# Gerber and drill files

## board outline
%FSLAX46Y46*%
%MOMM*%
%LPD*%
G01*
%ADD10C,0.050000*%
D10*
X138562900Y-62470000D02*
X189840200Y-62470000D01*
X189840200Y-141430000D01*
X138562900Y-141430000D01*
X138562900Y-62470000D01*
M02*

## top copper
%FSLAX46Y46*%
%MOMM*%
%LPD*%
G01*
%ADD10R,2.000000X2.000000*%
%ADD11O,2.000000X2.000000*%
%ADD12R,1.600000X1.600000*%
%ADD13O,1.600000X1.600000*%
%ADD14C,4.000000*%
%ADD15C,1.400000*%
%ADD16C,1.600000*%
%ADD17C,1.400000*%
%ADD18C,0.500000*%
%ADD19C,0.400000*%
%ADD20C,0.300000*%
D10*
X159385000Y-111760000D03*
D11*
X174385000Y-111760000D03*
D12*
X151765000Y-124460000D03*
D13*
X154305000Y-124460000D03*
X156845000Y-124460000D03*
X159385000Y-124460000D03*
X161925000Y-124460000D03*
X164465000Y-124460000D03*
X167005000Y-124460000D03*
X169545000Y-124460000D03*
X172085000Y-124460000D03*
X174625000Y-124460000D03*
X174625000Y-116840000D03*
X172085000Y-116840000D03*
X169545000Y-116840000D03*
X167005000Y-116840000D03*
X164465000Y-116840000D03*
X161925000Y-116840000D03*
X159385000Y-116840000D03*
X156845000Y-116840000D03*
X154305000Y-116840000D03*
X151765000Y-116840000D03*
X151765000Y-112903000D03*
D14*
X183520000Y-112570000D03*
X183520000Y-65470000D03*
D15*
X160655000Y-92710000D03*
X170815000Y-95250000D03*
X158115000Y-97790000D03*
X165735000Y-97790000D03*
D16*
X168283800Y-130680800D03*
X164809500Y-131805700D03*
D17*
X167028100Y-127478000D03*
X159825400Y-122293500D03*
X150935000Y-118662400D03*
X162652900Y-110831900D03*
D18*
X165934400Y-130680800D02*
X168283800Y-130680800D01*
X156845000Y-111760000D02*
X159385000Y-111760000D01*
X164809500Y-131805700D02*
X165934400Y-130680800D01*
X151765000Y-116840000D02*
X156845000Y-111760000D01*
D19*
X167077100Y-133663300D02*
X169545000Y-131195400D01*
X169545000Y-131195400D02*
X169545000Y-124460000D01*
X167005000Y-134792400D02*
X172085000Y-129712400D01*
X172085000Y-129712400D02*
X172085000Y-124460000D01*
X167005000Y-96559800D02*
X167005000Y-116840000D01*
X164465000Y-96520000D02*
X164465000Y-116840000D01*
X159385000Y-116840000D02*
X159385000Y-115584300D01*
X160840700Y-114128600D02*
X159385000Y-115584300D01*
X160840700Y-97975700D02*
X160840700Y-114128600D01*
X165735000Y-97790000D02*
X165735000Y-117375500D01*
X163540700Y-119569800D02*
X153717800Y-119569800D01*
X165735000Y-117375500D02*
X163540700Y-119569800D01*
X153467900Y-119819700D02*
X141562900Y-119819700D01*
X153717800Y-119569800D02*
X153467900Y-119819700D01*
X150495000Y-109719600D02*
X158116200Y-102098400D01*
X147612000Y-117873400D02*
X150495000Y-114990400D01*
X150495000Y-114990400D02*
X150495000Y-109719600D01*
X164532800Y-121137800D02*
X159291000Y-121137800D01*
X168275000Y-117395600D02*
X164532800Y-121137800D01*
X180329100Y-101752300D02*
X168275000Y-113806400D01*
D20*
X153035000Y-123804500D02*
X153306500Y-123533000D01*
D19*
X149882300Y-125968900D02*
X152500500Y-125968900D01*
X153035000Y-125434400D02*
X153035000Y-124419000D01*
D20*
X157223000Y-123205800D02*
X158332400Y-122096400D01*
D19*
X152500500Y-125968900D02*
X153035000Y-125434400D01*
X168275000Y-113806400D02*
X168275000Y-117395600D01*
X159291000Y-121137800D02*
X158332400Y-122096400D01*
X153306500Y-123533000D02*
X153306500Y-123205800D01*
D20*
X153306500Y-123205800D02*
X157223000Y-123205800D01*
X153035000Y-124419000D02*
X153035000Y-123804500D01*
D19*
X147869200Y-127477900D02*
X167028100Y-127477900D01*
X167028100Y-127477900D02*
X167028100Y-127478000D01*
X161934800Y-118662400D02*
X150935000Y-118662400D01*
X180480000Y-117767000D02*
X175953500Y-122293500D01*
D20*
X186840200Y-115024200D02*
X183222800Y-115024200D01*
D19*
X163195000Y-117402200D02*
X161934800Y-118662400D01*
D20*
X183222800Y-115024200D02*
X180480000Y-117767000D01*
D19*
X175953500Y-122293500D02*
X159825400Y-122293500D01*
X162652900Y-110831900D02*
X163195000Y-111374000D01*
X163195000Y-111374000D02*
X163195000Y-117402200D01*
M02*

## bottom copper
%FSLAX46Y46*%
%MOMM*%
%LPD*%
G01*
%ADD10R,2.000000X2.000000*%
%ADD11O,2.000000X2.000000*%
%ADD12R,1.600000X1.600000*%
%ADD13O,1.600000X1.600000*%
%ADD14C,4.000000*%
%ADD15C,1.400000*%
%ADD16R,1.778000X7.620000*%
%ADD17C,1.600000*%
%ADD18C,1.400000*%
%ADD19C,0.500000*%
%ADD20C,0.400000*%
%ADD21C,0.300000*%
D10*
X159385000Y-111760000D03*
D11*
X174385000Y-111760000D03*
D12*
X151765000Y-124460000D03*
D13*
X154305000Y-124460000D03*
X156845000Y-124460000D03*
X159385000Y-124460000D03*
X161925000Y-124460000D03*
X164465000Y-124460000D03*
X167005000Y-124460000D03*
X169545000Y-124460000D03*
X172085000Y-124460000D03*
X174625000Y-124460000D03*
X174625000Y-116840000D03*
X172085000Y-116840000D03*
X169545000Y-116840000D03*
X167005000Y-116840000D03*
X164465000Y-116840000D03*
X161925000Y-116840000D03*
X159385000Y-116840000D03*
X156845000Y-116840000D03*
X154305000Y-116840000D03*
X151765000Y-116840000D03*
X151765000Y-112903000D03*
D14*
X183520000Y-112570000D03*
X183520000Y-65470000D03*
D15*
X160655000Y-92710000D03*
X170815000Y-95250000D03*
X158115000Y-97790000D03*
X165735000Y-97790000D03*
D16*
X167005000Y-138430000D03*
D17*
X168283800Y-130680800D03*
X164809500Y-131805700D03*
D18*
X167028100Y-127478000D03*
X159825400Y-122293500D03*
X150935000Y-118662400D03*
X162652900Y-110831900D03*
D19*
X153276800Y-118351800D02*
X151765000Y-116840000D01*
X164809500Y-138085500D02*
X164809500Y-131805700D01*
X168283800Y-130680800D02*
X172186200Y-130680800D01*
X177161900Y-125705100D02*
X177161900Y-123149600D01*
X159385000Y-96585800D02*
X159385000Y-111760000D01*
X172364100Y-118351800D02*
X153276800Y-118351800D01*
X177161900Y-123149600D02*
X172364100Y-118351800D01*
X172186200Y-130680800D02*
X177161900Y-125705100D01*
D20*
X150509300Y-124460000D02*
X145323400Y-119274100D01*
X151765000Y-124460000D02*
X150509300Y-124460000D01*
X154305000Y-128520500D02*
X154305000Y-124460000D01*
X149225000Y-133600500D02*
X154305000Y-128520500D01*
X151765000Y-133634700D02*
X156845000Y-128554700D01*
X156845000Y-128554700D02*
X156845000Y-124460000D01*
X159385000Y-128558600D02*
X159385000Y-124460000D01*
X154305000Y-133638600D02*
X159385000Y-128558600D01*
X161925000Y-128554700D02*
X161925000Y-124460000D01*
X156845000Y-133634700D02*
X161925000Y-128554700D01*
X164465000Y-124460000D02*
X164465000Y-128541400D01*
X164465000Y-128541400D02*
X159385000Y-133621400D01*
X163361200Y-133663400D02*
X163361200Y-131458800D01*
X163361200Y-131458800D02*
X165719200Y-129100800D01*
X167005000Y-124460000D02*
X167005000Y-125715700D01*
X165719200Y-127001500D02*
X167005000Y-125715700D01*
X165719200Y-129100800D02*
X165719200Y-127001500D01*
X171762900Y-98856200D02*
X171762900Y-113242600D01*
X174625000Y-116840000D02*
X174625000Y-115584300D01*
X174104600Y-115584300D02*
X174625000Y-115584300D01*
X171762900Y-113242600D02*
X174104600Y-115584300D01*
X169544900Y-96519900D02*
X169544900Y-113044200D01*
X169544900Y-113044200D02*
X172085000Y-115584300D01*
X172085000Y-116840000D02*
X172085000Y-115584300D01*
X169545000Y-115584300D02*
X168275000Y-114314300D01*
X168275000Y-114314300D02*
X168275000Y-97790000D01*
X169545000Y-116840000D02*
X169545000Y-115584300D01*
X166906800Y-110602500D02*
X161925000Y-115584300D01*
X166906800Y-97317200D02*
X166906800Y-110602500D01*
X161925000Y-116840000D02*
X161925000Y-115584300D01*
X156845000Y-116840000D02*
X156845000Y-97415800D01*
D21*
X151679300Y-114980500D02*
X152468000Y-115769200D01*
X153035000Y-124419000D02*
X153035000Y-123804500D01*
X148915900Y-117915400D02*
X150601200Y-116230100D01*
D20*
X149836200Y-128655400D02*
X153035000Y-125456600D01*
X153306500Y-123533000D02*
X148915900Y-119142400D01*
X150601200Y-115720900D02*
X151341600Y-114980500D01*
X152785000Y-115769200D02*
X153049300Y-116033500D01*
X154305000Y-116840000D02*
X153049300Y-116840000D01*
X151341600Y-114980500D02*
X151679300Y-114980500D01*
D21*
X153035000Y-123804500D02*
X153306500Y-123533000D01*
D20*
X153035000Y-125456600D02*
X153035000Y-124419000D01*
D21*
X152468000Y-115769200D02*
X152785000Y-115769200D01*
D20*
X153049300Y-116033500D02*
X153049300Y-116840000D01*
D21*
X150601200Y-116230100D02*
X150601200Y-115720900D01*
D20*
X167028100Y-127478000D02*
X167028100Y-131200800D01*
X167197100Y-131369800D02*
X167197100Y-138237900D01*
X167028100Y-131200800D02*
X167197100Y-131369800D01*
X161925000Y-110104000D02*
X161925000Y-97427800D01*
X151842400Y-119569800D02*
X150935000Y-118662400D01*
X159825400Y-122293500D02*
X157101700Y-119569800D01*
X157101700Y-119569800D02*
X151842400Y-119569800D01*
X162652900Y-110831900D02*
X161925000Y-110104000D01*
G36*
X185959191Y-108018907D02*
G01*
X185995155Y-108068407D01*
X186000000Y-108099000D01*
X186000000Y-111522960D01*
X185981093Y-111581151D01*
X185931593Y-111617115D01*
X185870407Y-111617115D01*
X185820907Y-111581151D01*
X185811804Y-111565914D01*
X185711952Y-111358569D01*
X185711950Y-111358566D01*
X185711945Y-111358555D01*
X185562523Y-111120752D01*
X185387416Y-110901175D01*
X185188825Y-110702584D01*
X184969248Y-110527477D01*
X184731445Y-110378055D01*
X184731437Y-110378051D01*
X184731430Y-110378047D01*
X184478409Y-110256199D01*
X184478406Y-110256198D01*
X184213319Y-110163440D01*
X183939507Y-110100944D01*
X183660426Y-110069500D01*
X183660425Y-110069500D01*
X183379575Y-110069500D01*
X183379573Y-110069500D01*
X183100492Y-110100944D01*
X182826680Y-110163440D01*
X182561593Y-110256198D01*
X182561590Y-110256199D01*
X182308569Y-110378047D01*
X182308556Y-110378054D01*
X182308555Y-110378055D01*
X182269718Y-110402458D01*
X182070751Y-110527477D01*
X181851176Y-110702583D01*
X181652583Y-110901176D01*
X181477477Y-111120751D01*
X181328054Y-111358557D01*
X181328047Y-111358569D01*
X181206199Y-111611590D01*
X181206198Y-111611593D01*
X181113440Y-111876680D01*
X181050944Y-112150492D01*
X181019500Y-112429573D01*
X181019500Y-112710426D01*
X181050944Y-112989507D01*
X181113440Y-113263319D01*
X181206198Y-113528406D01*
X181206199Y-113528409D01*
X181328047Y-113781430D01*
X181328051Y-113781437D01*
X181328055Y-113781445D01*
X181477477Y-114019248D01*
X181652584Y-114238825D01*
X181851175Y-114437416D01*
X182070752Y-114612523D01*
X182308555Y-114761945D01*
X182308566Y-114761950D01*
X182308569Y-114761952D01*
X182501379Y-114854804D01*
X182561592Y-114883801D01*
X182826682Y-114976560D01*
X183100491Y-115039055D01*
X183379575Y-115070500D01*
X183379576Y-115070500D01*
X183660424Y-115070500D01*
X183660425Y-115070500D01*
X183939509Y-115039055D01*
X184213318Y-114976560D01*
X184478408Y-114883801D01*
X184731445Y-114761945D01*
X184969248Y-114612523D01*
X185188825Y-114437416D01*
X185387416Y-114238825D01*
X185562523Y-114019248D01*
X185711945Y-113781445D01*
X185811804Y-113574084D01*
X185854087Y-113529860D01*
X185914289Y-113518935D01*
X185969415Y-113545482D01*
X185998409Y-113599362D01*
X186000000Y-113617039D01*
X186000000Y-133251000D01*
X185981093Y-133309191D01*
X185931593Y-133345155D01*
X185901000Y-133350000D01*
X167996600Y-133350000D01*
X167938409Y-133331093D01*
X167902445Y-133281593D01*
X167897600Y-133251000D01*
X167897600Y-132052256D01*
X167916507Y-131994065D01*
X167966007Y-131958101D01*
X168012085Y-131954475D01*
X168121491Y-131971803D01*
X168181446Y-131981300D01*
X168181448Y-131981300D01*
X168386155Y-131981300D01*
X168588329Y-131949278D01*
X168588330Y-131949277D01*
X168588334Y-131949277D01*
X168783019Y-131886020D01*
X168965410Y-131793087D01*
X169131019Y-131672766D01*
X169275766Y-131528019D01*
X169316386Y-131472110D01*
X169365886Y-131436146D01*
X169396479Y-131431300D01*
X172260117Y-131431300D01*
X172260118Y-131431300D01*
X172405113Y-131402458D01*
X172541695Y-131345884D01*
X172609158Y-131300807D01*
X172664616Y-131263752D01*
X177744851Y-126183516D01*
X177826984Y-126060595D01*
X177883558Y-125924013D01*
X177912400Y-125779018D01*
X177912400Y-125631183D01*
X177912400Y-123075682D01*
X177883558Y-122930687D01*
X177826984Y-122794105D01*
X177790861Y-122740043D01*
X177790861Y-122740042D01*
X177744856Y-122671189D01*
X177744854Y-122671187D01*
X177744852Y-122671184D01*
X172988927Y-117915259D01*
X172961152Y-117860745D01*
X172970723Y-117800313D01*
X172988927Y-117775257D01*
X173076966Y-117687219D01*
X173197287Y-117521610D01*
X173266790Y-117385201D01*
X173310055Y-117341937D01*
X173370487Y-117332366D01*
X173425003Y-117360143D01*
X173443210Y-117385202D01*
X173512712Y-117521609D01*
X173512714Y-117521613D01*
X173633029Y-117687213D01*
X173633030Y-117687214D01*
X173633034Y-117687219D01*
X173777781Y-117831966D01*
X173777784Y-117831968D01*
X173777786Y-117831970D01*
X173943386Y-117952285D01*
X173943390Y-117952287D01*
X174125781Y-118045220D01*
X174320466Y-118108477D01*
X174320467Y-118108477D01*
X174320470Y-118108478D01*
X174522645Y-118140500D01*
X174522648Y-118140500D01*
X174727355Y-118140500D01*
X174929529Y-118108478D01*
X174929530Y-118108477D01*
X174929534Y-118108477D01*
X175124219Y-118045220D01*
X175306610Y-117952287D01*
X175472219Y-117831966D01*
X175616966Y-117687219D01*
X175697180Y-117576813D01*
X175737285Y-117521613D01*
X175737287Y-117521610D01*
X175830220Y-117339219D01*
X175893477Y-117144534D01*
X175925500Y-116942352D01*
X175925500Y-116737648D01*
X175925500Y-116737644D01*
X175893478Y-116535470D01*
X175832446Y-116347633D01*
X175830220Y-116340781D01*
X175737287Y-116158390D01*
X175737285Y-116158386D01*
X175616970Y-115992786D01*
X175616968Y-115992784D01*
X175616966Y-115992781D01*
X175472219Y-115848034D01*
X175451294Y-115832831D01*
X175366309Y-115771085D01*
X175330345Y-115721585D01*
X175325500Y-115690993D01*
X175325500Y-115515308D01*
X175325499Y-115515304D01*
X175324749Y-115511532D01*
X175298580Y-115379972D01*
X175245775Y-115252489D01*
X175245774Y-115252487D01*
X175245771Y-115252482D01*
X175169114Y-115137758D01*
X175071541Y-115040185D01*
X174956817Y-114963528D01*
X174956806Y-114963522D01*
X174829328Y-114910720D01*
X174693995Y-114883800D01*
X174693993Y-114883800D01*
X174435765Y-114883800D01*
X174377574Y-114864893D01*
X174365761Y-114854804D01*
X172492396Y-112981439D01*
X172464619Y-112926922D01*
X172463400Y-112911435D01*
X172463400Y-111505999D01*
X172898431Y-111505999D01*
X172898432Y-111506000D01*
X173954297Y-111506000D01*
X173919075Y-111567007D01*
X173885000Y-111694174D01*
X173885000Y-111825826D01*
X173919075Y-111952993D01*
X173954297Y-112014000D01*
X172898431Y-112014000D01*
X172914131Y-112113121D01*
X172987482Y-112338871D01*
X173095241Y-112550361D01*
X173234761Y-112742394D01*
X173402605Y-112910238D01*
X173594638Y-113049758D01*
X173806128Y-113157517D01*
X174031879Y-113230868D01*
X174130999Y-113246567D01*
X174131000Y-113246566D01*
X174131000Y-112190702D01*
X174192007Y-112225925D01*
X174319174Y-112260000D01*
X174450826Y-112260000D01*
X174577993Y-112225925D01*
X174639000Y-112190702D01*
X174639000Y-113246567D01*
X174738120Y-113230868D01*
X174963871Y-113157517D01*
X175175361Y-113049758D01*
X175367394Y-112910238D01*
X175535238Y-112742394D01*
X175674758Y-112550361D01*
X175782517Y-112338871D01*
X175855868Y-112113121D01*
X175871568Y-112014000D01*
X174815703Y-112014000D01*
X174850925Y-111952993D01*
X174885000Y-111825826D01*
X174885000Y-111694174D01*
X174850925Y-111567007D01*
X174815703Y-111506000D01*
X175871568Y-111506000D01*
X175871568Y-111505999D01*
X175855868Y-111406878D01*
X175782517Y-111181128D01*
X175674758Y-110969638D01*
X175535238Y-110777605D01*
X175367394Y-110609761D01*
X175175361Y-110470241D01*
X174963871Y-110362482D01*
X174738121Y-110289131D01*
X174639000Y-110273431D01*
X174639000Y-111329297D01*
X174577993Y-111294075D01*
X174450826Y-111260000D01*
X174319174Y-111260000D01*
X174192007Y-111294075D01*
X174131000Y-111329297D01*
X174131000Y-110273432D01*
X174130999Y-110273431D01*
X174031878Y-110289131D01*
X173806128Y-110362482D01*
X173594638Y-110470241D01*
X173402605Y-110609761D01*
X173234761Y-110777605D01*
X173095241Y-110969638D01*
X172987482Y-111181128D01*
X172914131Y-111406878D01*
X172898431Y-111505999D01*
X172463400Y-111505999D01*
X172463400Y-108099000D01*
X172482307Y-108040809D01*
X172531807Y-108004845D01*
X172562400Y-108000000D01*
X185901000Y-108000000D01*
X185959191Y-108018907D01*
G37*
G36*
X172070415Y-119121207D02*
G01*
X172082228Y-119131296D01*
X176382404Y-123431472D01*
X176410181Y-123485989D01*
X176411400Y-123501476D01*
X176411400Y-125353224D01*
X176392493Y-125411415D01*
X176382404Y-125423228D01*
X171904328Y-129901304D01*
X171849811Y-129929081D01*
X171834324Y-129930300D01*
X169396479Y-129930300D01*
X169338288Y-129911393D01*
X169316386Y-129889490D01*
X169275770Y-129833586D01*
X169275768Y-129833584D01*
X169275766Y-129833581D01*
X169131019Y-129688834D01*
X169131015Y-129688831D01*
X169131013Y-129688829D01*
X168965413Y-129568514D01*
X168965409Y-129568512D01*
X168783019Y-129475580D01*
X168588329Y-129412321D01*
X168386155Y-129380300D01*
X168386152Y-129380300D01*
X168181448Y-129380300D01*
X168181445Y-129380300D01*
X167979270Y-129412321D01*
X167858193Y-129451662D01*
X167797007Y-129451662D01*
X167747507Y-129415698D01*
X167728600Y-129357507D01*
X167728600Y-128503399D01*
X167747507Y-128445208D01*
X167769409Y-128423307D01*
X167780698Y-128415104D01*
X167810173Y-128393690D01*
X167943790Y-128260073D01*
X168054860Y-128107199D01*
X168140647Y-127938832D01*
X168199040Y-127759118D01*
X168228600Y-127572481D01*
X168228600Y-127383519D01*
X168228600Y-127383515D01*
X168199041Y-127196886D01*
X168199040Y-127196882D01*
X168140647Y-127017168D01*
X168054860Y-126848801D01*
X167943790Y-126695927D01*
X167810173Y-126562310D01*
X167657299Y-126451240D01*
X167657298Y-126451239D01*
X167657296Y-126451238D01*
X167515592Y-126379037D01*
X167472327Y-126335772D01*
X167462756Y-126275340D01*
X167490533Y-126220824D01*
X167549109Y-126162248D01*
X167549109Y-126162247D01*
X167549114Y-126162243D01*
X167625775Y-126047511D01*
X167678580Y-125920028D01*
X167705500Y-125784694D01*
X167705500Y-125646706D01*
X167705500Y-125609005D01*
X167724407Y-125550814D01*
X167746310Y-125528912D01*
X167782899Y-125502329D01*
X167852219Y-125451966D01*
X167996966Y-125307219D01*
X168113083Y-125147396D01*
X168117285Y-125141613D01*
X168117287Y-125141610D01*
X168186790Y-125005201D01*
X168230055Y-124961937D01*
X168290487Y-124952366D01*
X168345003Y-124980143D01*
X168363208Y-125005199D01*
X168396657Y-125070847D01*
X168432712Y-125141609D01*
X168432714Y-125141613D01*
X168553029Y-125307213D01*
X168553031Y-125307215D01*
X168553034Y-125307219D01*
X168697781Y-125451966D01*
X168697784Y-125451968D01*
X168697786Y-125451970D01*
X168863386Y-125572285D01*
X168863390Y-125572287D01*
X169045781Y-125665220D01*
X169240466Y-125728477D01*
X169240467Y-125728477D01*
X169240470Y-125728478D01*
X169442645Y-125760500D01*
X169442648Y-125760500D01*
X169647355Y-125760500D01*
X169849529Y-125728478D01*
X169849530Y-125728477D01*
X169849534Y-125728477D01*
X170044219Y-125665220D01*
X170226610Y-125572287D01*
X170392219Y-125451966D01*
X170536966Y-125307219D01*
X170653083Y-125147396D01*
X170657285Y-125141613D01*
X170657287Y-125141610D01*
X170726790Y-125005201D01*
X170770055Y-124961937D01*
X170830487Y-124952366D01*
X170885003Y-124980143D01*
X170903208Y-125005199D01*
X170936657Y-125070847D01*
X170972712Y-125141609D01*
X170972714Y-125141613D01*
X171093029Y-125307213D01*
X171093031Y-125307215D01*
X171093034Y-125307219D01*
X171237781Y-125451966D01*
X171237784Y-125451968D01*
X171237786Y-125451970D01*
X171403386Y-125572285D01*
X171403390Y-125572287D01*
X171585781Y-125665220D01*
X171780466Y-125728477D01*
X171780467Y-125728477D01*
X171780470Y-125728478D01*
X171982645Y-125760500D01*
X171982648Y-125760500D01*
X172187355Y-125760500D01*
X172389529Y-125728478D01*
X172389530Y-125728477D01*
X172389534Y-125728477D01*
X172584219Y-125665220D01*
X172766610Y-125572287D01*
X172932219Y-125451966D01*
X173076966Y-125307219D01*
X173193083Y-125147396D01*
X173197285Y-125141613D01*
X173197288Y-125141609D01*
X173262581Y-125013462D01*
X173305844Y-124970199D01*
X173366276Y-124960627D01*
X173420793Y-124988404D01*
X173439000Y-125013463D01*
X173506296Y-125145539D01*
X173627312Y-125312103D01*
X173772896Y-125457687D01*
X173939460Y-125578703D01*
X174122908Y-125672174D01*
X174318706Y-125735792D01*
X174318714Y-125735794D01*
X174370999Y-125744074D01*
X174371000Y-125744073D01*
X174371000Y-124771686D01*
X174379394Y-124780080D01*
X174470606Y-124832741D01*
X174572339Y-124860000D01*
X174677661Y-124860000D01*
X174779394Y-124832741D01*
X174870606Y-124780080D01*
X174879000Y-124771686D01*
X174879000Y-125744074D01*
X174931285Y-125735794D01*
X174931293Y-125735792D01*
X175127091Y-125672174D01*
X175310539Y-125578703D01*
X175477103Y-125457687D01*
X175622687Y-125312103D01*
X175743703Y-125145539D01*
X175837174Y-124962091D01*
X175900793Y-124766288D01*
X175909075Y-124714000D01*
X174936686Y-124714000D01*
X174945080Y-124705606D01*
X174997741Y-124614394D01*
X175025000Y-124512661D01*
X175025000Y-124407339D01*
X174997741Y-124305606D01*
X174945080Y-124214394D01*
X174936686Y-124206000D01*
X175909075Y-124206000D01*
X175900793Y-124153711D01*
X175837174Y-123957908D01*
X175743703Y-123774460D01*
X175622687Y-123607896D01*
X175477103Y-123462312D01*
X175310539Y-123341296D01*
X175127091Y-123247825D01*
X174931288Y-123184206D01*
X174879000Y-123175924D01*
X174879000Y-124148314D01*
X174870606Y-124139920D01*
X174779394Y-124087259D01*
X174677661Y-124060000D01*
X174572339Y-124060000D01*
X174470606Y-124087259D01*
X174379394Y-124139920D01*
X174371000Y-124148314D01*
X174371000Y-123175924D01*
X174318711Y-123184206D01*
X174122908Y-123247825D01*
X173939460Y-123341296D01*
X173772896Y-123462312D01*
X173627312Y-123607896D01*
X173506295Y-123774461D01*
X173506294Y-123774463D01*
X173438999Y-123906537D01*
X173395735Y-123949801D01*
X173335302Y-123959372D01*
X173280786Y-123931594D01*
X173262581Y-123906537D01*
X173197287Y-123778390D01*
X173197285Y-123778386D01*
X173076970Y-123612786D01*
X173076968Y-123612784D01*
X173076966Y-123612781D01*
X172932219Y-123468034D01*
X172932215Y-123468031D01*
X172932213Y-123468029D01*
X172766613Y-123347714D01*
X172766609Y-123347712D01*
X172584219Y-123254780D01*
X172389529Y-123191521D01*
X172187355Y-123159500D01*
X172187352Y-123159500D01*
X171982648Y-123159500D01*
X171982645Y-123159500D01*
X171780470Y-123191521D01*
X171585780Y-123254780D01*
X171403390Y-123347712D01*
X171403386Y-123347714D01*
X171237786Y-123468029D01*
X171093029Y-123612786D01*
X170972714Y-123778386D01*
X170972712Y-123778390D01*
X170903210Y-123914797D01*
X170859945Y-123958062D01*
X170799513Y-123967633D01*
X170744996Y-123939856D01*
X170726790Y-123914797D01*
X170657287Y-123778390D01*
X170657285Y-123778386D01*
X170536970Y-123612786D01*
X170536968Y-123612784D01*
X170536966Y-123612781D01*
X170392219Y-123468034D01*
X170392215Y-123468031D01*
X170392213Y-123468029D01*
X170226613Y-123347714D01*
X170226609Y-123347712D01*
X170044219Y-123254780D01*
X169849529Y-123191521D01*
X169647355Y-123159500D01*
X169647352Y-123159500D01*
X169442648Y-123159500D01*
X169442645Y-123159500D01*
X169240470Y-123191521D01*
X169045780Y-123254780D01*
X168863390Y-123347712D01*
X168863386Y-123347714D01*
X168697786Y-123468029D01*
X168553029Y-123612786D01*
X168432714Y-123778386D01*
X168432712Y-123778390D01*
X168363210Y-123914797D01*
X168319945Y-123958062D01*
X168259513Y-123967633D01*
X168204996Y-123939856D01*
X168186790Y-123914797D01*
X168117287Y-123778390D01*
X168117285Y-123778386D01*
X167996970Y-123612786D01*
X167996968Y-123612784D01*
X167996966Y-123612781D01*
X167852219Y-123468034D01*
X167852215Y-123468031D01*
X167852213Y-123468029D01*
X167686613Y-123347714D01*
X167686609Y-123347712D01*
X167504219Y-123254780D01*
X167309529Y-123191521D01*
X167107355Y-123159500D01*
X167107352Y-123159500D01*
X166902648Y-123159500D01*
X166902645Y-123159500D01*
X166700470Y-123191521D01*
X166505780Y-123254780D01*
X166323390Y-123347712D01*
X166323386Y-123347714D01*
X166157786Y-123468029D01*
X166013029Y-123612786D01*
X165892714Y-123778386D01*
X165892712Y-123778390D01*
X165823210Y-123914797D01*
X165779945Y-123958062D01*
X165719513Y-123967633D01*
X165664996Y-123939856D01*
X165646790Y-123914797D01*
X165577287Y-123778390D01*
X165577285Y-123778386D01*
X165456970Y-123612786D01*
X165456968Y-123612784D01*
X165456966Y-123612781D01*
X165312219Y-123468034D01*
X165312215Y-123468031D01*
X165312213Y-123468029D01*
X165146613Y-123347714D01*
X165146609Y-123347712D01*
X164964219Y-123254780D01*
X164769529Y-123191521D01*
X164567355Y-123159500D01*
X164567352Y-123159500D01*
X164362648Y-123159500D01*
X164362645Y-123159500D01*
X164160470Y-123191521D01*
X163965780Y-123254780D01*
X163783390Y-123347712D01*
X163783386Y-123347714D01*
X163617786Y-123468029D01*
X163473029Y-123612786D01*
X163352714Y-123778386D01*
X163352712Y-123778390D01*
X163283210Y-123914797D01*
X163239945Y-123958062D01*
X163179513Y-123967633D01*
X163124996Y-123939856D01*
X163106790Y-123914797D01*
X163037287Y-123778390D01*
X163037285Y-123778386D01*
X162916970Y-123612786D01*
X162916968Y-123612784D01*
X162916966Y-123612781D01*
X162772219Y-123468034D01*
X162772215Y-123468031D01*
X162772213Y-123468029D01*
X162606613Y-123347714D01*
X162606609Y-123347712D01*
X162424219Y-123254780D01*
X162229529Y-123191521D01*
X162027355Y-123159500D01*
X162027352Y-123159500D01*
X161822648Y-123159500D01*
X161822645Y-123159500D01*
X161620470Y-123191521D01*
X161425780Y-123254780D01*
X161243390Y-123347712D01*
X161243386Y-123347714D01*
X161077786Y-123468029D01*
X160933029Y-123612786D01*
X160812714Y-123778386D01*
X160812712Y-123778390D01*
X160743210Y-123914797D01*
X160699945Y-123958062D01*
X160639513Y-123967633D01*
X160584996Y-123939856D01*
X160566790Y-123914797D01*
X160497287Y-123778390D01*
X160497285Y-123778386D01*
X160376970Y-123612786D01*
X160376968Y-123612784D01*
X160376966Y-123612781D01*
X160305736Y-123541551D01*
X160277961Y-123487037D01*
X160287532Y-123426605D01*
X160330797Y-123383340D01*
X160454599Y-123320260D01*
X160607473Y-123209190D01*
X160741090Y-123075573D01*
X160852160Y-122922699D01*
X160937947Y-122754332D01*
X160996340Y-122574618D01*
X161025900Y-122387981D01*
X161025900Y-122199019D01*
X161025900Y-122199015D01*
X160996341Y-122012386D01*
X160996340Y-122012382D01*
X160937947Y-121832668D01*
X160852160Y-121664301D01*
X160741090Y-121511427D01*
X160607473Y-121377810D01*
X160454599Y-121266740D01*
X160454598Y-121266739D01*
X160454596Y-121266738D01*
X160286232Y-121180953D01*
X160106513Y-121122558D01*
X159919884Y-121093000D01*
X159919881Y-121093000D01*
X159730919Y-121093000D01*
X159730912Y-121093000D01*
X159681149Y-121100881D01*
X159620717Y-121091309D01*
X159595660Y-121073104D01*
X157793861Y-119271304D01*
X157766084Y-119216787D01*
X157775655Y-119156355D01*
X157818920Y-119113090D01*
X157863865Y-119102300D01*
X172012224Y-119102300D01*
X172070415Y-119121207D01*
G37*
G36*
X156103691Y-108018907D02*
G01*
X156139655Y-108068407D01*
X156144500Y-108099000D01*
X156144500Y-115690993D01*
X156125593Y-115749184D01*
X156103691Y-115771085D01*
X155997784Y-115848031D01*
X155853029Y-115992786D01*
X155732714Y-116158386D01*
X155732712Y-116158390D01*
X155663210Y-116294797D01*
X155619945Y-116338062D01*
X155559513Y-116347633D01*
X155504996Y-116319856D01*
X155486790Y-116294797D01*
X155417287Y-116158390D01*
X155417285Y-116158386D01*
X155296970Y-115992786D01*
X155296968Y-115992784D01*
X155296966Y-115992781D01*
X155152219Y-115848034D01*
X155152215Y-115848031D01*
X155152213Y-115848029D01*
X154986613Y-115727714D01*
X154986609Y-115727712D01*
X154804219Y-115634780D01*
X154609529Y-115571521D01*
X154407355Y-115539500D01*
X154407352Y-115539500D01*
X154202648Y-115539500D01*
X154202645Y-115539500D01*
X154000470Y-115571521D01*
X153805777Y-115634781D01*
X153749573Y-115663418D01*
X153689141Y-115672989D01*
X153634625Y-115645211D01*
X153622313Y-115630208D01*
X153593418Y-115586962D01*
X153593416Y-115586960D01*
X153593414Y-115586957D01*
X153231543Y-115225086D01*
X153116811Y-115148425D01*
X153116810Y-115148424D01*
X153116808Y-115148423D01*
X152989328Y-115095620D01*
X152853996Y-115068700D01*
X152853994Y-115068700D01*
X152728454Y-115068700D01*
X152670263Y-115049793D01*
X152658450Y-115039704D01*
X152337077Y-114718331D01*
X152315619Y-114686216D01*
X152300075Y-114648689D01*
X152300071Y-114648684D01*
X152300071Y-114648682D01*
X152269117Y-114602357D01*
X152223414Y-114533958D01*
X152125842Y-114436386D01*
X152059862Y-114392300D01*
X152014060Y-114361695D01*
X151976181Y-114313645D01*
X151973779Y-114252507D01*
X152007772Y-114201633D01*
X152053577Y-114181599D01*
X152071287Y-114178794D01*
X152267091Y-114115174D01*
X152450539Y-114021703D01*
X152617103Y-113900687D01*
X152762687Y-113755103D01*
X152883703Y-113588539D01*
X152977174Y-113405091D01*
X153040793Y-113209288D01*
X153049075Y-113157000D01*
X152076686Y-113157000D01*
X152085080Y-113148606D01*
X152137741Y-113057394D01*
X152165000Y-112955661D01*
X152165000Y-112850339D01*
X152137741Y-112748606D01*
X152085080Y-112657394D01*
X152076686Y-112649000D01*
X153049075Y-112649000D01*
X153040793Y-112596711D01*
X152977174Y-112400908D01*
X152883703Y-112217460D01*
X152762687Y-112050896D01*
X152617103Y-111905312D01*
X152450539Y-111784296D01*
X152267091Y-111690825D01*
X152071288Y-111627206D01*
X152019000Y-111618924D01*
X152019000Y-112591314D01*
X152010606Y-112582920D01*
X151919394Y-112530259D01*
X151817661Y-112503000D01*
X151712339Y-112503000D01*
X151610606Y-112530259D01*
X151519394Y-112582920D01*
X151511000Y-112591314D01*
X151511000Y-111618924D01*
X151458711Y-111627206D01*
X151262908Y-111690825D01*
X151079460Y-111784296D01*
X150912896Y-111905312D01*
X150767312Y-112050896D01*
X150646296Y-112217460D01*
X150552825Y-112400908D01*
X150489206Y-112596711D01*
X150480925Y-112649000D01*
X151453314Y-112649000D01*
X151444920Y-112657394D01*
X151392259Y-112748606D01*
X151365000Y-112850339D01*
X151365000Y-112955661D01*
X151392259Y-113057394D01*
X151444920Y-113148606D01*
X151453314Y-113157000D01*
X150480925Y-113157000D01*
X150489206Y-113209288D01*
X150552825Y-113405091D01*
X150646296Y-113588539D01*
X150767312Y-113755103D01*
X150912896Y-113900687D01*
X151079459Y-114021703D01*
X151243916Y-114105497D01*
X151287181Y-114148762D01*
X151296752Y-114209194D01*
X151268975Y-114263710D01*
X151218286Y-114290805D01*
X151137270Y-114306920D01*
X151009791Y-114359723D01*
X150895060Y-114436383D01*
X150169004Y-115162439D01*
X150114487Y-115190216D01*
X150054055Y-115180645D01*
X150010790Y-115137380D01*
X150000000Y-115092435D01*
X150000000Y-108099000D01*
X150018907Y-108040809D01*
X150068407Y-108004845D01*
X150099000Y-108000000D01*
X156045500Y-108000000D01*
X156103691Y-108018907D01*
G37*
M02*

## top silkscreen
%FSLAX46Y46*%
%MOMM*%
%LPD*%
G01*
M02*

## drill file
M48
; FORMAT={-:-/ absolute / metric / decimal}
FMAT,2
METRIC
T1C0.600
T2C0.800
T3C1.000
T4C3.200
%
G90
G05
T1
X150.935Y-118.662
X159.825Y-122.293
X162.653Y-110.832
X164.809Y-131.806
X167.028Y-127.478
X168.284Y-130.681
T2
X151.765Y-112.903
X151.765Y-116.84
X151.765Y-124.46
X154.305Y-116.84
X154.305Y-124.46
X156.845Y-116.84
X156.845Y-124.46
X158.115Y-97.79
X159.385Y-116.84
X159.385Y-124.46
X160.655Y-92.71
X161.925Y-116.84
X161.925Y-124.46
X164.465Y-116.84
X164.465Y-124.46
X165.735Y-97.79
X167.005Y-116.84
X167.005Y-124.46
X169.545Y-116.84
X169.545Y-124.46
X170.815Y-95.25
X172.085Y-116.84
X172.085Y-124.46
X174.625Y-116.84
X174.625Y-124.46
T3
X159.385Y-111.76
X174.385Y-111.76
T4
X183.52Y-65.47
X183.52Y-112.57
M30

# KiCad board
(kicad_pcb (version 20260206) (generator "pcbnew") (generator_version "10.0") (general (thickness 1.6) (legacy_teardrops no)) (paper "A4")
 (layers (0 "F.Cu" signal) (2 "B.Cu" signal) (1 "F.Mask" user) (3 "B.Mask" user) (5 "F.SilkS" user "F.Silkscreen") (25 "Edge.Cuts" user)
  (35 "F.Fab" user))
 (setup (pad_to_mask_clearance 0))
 (gr_rect (start 138.5629 62.47) (end 189.8402 141.43) (stroke (width 0.05) (type default)) (fill no) (layer "Edge.Cuts"))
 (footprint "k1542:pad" (layer "F.Cu") (at 159.385 111.76 0.0)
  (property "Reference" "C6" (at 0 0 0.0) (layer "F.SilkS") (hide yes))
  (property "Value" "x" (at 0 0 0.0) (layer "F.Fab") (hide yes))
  (pad "1" thru_hole rect (at 0 0 0.0) (size 2.0 2.0) (drill 1.0) (layers "*.Cu" "*.Mask") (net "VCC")))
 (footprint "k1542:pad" (layer "F.Cu") (at 174.385 111.76 0.0)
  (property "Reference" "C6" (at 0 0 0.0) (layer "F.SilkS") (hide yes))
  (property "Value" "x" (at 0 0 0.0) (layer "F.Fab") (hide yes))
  (pad "2" thru_hole oval (at 0 0 0.0) (size 2.0 2.0) (drill 1.0) (layers "*.Cu" "*.Mask") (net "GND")))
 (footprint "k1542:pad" (layer "F.Cu") (at 151.765 124.46 90.0)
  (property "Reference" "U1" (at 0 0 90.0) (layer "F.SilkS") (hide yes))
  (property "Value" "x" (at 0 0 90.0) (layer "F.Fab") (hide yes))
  (pad "1" thru_hole rect (at 0 0 90.0) (size 1.6 1.6) (drill 0.8) (layers "*.Cu" "*.Mask") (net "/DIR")))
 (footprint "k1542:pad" (layer "F.Cu") (at 154.305 124.46 90.0)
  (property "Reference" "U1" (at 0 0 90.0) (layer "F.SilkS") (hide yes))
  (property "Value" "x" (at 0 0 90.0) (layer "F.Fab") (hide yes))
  (pad "2" thru_hole oval (at 0 0 90.0) (size 1.6 1.6) (drill 0.8) (layers "*.Cu" "*.Mask") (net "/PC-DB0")))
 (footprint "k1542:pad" (layer "F.Cu") (at 156.845 124.46 90.0)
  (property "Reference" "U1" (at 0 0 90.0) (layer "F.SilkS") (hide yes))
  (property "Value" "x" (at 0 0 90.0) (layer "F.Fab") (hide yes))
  (pad "3" thru_hole oval (at 0 0 90.0) (size 1.6 1.6) (drill 0.8) (layers "*.Cu" "*.Mask") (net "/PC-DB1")))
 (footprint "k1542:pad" (layer "F.Cu") (at 159.385 124.46 90.0)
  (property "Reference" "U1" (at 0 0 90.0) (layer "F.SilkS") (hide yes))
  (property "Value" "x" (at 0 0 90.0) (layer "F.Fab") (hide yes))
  (pad "4" thru_hole oval (at 0 0 90.0) (size 1.6 1.6) (drill 0.8) (layers "*.Cu" "*.Mask") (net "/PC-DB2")))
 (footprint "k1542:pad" (layer "F.Cu") (at 161.925 124.46 90.0)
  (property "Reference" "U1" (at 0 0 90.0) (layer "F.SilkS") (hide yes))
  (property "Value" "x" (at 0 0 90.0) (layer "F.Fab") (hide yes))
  (pad "5" thru_hole oval (at 0 0 90.0) (size 1.6 1.6) (drill 0.8) (layers "*.Cu" "*.Mask") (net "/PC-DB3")))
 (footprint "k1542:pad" (layer "F.Cu") (at 164.465 124.46 90.0)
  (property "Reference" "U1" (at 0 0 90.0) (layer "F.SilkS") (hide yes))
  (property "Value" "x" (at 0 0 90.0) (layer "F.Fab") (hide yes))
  (pad "6" thru_hole oval (at 0 0 90.0) (size 1.6 1.6) (drill 0.8) (layers "*.Cu" "*.Mask") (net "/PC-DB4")))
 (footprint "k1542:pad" (layer "F.Cu") (at 167.005 124.46 90.0)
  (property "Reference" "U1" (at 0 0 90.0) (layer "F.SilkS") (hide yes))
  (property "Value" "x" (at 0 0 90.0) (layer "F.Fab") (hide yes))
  (pad "7" thru_hole oval (at 0 0 90.0) (size 1.6 1.6) (drill 0.8) (layers "*.Cu" "*.Mask") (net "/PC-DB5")))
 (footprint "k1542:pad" (layer "F.Cu") (at 169.545 124.46 90.0)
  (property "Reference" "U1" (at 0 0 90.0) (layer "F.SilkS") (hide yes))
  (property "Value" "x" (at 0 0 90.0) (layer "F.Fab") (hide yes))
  (pad "8" thru_hole oval (at 0 0 90.0) (size 1.6 1.6) (drill 0.8) (layers "*.Cu" "*.Mask") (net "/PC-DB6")))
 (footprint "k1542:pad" (layer "F.Cu") (at 172.085 124.46 90.0)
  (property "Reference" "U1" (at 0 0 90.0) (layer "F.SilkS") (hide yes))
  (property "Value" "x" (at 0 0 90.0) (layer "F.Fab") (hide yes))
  (pad "9" thru_hole oval (at 0 0 90.0) (size 1.6 1.6) (drill 0.8) (layers "*.Cu" "*.Mask") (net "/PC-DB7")))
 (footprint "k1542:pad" (layer "F.Cu") (at 174.625 124.46 90.0)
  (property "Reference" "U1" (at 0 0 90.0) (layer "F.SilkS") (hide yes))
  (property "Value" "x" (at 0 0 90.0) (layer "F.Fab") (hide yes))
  (pad "10" thru_hole oval (at 0 0 90.0) (size 1.6 1.6) (drill 0.8) (layers "*.Cu" "*.Mask") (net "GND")))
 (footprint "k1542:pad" (layer "F.Cu") (at 174.625 116.84 90.0)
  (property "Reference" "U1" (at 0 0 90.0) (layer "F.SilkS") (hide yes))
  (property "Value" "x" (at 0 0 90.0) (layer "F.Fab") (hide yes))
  (pad "11" thru_hole oval (at 0 0 90.0) (size 1.6 1.6) (drill 0.8) (layers "*.Cu" "*.Mask") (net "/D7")))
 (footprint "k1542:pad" (layer "F.Cu") (at 172.085 116.84 90.0)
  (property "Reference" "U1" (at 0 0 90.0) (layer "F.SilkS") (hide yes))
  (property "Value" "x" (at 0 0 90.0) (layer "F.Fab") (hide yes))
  (pad "12" thru_hole oval (at 0 0 90.0) (size 1.6 1.6) (drill 0.8) (layers "*.Cu" "*.Mask") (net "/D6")))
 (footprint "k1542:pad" (layer "F.Cu") (at 169.545 116.84 90.0)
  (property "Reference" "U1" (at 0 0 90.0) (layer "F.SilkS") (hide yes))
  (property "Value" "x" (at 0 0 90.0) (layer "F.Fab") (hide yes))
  (pad "13" thru_hole oval (at 0 0 90.0) (size 1.6 1.6) (drill 0.8) (layers "*.Cu" "*.Mask") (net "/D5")))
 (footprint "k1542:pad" (layer "F.Cu") (at 167.005 116.84 90.0)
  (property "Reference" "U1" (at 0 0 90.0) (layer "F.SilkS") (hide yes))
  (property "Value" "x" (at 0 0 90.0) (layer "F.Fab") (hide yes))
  (pad "14" thru_hole oval (at 0 0 90.0) (size 1.6 1.6) (drill 0.8) (layers "*.Cu" "*.Mask") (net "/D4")))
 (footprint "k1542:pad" (layer "F.Cu") (at 164.465 116.84 90.0)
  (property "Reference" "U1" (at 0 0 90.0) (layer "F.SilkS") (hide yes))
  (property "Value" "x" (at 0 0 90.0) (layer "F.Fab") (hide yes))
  (pad "15" thru_hole oval (at 0 0 90.0) (size 1.6 1.6) (drill 0.8) (layers "*.Cu" "*.Mask") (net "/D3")))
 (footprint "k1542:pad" (layer "F.Cu") (at 161.925 116.84 90.0)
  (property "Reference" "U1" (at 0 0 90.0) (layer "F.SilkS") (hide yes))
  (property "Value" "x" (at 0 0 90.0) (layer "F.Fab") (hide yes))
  (pad "16" thru_hole oval (at 0 0 90.0) (size 1.6 1.6) (drill 0.8) (layers "*.Cu" "*.Mask") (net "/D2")))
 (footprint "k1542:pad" (layer "F.Cu") (at 159.385 116.84 90.0)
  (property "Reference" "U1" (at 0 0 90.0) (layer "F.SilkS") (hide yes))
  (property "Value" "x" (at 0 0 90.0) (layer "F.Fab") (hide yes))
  (pad "17" thru_hole oval (at 0 0 90.0) (size 1.6 1.6) (drill 0.8) (layers "*.Cu" "*.Mask") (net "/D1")))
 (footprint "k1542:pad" (layer "F.Cu") (at 156.845 116.84 90.0)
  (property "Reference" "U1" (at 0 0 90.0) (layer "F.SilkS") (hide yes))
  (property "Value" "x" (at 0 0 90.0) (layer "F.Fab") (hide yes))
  (pad "18" thru_hole oval (at 0 0 90.0) (size 1.6 1.6) (drill 0.8) (layers "*.Cu" "*.Mask") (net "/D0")))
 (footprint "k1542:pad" (layer "F.Cu") (at 154.305 116.84 90.0)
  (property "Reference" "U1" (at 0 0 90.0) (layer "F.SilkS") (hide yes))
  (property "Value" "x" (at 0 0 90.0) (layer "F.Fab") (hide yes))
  (pad "19" thru_hole oval (at 0 0 90.0) (size 1.6 1.6) (drill 0.8) (layers "*.Cu" "*.Mask") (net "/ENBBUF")))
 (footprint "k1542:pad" (layer "F.Cu") (at 151.765 116.84 90.0)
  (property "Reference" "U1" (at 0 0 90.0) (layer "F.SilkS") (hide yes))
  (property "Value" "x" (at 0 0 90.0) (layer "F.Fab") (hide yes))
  (pad "20" thru_hole oval (at 0 0 90.0) (size 1.6 1.6) (drill 0.8) (layers "*.Cu" "*.Mask") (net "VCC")))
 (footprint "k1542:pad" (layer "F.Cu") (at 151.765 112.903 90.0)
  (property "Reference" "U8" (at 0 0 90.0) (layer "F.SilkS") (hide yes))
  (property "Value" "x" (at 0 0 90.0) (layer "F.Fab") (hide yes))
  (pad "12" thru_hole oval (at 0 0 90.0) (size 1.6 1.6) (drill 0.8) (layers "*.Cu" "*.Mask") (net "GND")))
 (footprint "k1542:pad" (layer "F.Cu") (at 183.52 112.57 90.0)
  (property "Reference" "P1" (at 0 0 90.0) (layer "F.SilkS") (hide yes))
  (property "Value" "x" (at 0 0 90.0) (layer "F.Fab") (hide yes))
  (pad "0" thru_hole circle (at 0 0 90.0) (size 4.0 4.0) (drill 3.2) (layers "*.Cu" "*.Mask") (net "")))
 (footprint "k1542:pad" (layer "F.Cu") (at 183.52 65.47 90.0)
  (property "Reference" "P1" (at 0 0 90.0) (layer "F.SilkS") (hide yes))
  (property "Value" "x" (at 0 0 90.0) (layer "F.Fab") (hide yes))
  (pad "0" thru_hole circle (at 0 0 90.0) (size 4.0 4.0) (drill 3.2) (layers "*.Cu" "*.Mask") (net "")))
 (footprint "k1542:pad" (layer "F.Cu") (at 160.655 92.71 180.0)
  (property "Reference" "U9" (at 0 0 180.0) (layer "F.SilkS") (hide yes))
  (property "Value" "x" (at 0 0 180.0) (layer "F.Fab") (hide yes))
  (pad "L8" thru_hole circle (at 0 0 180.0) (size 1.4 1.4) (drill 0.8) (layers "*.Cu" "*.Mask") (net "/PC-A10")))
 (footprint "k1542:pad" (layer "F.Cu") (at 170.815 95.25 180.0)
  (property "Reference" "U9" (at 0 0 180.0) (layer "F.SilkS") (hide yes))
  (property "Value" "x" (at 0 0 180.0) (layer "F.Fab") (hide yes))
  (pad "M12" thru_hole circle (at 0 0 180.0) (size 1.4 1.4) (drill 0.8) (layers "*.Cu" "*.Mask") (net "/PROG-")))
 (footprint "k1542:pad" (layer "F.Cu") (at 158.115 97.79 180.0)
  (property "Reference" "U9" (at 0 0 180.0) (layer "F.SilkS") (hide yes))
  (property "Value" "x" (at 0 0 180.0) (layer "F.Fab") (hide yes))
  (pad "N7" thru_hole circle (at 0 0 180.0) (size 1.4 1.4) (drill 0.8) (layers "*.Cu" "*.Mask") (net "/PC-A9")))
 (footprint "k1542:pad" (layer "F.Cu") (at 165.735 97.79 180.0)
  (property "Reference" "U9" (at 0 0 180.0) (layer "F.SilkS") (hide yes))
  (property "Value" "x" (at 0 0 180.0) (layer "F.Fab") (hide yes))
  (pad "N10" thru_hole circle (at 0 0 180.0) (size 1.4 1.4) (drill 0.8) (layers "*.Cu" "*.Mask") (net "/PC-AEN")))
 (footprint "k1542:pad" (layer "F.Cu") (at 167.005 138.43 0.0)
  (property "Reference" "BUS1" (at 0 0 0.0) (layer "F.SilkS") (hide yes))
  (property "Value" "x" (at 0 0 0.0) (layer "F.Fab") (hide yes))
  (pad "2" smd rect (at 0 0 0.0) (size 1.778 7.62) (layers "B.Cu" "B.Mask") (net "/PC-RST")))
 (via locked (at 168.2838 130.6808) (size 1.6) (drill 0.6) (layers "F.Cu" "B.Cu") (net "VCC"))
 (via locked (at 164.8095 131.8057) (size 1.6) (drill 0.6) (layers "F.Cu" "B.Cu") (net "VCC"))
 (via locked (at 167.0281 127.478) (size 1.4) (drill 0.6) (layers "F.Cu" "B.Cu") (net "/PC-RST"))
 (via locked (at 159.8254 122.2935) (size 1.4) (drill 0.6) (layers "F.Cu" "B.Cu") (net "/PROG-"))
 (via locked (at 150.935 118.6624) (size 1.4) (drill 0.6) (layers "F.Cu" "B.Cu") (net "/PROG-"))
 (via locked (at 162.6529 110.8319) (size 1.4) (drill 0.6) (layers "F.Cu" "B.Cu") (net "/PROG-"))
 (segment locked (start 165.9344 130.6808) (end 168.2838 130.6808) (width 0.5) (layer "F.Cu") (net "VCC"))
 (segment locked (start 156.845 111.76) (end 159.385 111.76) (width 0.5) (layer "F.Cu") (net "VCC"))
 (segment locked (start 164.8095 131.8057) (end 165.9344 130.6808) (width 0.5) (layer "F.Cu") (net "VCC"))
 (segment locked (start 151.765 116.84) (end 156.845 111.76) (width 0.5) (layer "F.Cu") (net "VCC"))
 (segment locked (start 153.2768 118.3518) (end 151.765 116.84) (width 0.5) (layer "B.Cu") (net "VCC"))
 (segment locked (start 164.8095 138.0855) (end 164.8095 131.8057) (width 0.5) (layer "B.Cu") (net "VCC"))
 (segment locked (start 168.2838 130.6808) (end 172.1862 130.6808) (width 0.5) (layer "B.Cu") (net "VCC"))
 (segment locked (start 177.1619 125.7051) (end 177.1619 123.1496) (width 0.5) (layer "B.Cu") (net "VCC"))
 (segment locked (start 159.385 96.5858) (end 159.385 111.76) (width 0.5) (layer "B.Cu") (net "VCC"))
 (segment locked (start 172.3641 118.3518) (end 153.2768 118.3518) (width 0.5) (layer "B.Cu") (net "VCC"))
 (segment locked (start 177.1619 123.1496) (end 172.3641 118.3518) (width 0.5) (layer "B.Cu") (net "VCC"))
 (segment locked (start 172.1862 130.6808) (end 177.1619 125.7051) (width 0.5) (layer "B.Cu") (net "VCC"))
 (segment locked (start 150.5093 124.46) (end 145.3234 119.2741) (width 0.4) (layer "B.Cu") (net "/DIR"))
 (segment locked (start 151.765 124.46) (end 150.5093 124.46) (width 0.4) (layer "B.Cu") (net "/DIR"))
 (segment locked (start 154.305 128.5205) (end 154.305 124.46) (width 0.4) (layer "B.Cu") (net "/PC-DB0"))
 (segment locked (start 149.225 133.6005) (end 154.305 128.5205) (width 0.4) (layer "B.Cu") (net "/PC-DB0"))
 (segment locked (start 151.765 133.6347) (end 156.845 128.5547) (width 0.4) (layer "B.Cu") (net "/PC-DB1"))
 (segment locked (start 156.845 128.5547) (end 156.845 124.46) (width 0.4) (layer "B.Cu") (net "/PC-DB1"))
 (segment locked (start 159.385 128.5586) (end 159.385 124.46) (width 0.4) (layer "B.Cu") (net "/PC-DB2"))
 (segment locked (start 154.305 133.6386) (end 159.385 128.5586) (width 0.4) (layer "B.Cu") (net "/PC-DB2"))
 (segment locked (start 161.925 128.5547) (end 161.925 124.46) (width 0.4) (layer "B.Cu") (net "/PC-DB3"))
 (segment locked (start 156.845 133.6347) (end 161.925 128.5547) (width 0.4) (layer "B.Cu") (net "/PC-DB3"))
 (segment locked (start 164.465 124.46) (end 164.465 128.5414) (width 0.4) (layer "B.Cu") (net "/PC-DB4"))
 (segment locked (start 164.465 128.5414) (end 159.385 133.6214) (width 0.4) (layer "B.Cu") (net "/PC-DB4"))
 (segment locked (start 163.3612 133.6634) (end 163.3612 131.4588) (width 0.4) (layer "B.Cu") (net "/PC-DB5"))
 (segment locked (start 163.3612 131.4588) (end 165.7192 129.1008) (width 0.4) (layer "B.Cu") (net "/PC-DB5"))
 (segment locked (start 167.005 124.46) (end 167.005 125.7157) (width 0.4) (layer "B.Cu") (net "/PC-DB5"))
 (segment locked (start 165.7192 127.0015) (end 167.005 125.7157) (width 0.4) (layer "B.Cu") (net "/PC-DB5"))
 (segment locked (start 165.7192 129.1008) (end 165.7192 127.0015) (width 0.4) (layer "B.Cu") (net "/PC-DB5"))
 (segment locked (start 167.0771 133.6633) (end 169.545 131.1954) (width 0.4) (layer "F.Cu") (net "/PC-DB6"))
 (segment locked (start 169.545 131.1954) (end 169.545 124.46) (width 0.4) (layer "F.Cu") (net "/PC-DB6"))
 (segment locked (start 167.005 134.7924) (end 172.085 129.7124) (width 0.4) (layer "F.Cu") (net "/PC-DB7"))
 (segment locked (start 172.085 129.7124) (end 172.085 124.46) (width 0.4) (layer "F.Cu") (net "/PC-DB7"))
 (segment locked (start 171.7629 98.8562) (end 171.7629 113.2426) (width 0.4) (layer "B.Cu") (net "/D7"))
 (segment locked (start 174.625 116.84) (end 174.625 115.5843) (width 0.4) (layer "B.Cu") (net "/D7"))
 (segment locked (start 174.1046 115.5843) (end 174.625 115.5843) (width 0.4) (layer "B.Cu") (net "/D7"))
 (segment locked (start 171.7629 113.2426) (end 174.1046 115.5843) (width 0.4) (layer "B.Cu") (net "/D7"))
 (segment locked (start 169.5449 96.5199) (end 169.5449 113.0442) (width 0.4) (layer "B.Cu") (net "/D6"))
 (segment locked (start 169.5449 113.0442) (end 172.085 115.5843) (width 0.4) (layer "B.Cu") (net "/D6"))
 (segment locked (start 172.085 116.84) (end 172.085 115.5843) (width 0.4) (layer "B.Cu") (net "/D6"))
 (segment locked (start 169.545 115.5843) (end 168.275 114.3143) (width 0.4) (layer "B.Cu") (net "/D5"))
 (segment locked (start 168.275 114.3143) (end 168.275 97.79) (width 0.4) (layer "B.Cu") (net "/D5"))
 (segment locked (start 169.545 116.84) (end 169.545 115.5843) (width 0.4) (layer "B.Cu") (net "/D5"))
 (segment locked (start 167.005 96.5598) (end 167.005 116.84) (width 0.4) (layer "F.Cu") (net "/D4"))
 (segment locked (start 164.465 96.52) (end 164.465 116.84) (width 0.4) (layer "F.Cu") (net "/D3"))
 (segment locked (start 166.9068 110.6025) (end 161.925 115.5843) (width 0.4) (layer "B.Cu") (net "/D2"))
 (segment locked (start 166.9068 97.3172) (end 166.9068 110.6025) (width 0.4) (layer "B.Cu") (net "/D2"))
 (segment locked (start 161.925 116.84) (end 161.925 115.5843) (width 0.4) (layer "B.Cu") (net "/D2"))
 (segment locked (start 159.385 116.84) (end 159.385 115.5843) (width 0.4) (layer "F.Cu") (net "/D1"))
 (segment locked (start 160.8407 114.1286) (end 159.385 115.5843) (width 0.4) (layer "F.Cu") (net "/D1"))
 (segment locked (start 160.8407 97.9757) (end 160.8407 114.1286) (width 0.4) (layer "F.Cu") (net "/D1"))
 (segment locked (start 156.845 116.84) (end 156.845 97.4158) (width 0.4) (layer "B.Cu") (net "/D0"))
 (segment locked (start 151.6793 114.9805) (end 152.468 115.7692) (width 0.3) (layer "B.Cu") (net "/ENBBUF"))
 (segment locked (start 153.035 124.419) (end 153.035 123.8045) (width 0.3) (layer "B.Cu") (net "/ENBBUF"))
 (segment locked (start 148.9159 117.9154) (end 150.6012 116.2301) (width 0.3) (layer "B.Cu") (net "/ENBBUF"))
 (segment locked (start 149.8362 128.6554) (end 153.035 125.4566) (width 0.4) (layer "B.Cu") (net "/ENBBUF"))
 (segment locked (start 153.3065 123.533) (end 148.9159 119.1424) (width 0.4) (layer "B.Cu") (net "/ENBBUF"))
 (segment locked (start 150.6012 115.7209) (end 151.3416 114.9805) (width 0.4) (layer "B.Cu") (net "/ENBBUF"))
 (segment locked (start 152.785 115.7692) (end 153.0493 116.0335) (width 0.4) (layer "B.Cu") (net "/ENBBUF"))
 (segment locked (start 154.305 116.84) (end 153.0493 116.84) (width 0.4) (layer "B.Cu") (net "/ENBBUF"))
 (segment locked (start 151.3416 114.9805) (end 151.6793 114.9805) (width 0.4) (layer "B.Cu") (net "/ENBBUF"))
 (segment locked (start 153.035 123.8045) (end 153.3065 123.533) (width 0.3) (layer "B.Cu") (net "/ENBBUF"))
 (segment locked (start 153.035 125.4566) (end 153.035 124.419) (width 0.4) (layer "B.Cu") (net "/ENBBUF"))
 (segment locked (start 152.468 115.7692) (end 152.785 115.7692) (width 0.3) (layer "B.Cu") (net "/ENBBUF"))
 (segment locked (start 153.0493 116.0335) (end 153.0493 116.84) (width 0.4) (layer "B.Cu") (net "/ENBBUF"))
 (segment locked (start 150.6012 116.2301) (end 150.6012 115.7209) (width 0.3) (layer "B.Cu") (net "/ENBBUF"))
 (segment locked (start 165.735 97.79) (end 165.735 117.3755) (width 0.4) (layer "F.Cu") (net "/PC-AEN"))
 (segment locked (start 163.5407 119.5698) (end 153.7178 119.5698) (width 0.4) (layer "F.Cu") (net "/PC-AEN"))
 (segment locked (start 165.735 117.3755) (end 163.5407 119.5698) (width 0.4) (layer "F.Cu") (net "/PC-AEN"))
 (segment locked (start 153.4679 119.8197) (end 141.5629 119.8197) (width 0.4) (layer "F.Cu") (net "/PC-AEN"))
 (segment locked (start 153.7178 119.5698) (end 153.4679 119.8197) (width 0.4) (layer "F.Cu") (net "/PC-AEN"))
 (segment locked (start 150.495 109.7196) (end 158.1162 102.0984) (width 0.4) (layer "F.Cu") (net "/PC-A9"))
 (segment locked (start 147.612 117.8734) (end 150.495 114.9904) (width 0.4) (layer "F.Cu") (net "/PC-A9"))
 (segment locked (start 150.495 114.9904) (end 150.495 109.7196) (width 0.4) (layer "F.Cu") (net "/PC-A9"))
 (segment locked (start 164.5328 121.1378) (end 159.291 121.1378) (width 0.4) (layer "F.Cu") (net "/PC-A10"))
 (segment locked (start 168.275 117.3956) (end 164.5328 121.1378) (width 0.4) (layer "F.Cu") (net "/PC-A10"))
 (segment locked (start 180.3291 101.7523) (end 168.275 113.8064) (width 0.4) (layer "F.Cu") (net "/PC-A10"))
 (segment locked (start 153.035 123.8045) (end 153.3065 123.533) (width 0.3) (layer "F.Cu") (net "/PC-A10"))
 (segment locked (start 149.8823 125.9689) (end 152.5005 125.9689) (width 0.4) (layer "F.Cu") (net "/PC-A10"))
 (segment locked (start 153.035 125.4344) (end 153.035 124.419) (width 0.4) (layer "F.Cu") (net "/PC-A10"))
 (segment locked (start 157.223 123.2058) (end 158.3324 122.0964) (width 0.3) (layer "F.Cu") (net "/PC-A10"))
 (segment locked (start 152.5005 125.9689) (end 153.035 125.4344) (width 0.4) (layer "F.Cu") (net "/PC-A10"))
 (segment locked (start 168.275 113.8064) (end 168.275 117.3956) (width 0.4) (layer "F.Cu") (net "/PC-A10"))
 (segment locked (start 159.291 121.1378) (end 158.3324 122.0964) (width 0.4) (layer "F.Cu") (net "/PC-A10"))
 (segment locked (start 153.3065 123.533) (end 153.3065 123.2058) (width 0.4) (layer "F.Cu") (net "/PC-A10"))
 (segment locked (start 153.3065 123.2058) (end 157.223 123.2058) (width 0.3) (layer "F.Cu") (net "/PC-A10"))
 (segment locked (start 153.035 124.419) (end 153.035 123.8045) (width 0.3) (layer "F.Cu") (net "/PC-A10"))
 (segment locked (start 147.8692 127.4779) (end 167.0281 127.4779) (width 0.4) (layer "F.Cu") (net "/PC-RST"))
 (segment locked (start 167.0281 127.4779) (end 167.0281 127.478) (width 0.4) (layer "F.Cu") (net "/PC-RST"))
 (segment locked (start 167.0281 127.478) (end 167.0281 131.2008) (width 0.4) (layer "B.Cu") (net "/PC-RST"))
 (segment locked (start 167.1971 131.3698) (end 167.1971 138.2379) (width 0.4) (layer "B.Cu") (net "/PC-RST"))
 (segment locked (start 167.0281 131.2008) (end 167.1971 131.3698) (width 0.4) (layer "B.Cu") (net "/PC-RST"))
 (segment locked (start 161.9348 118.6624) (end 150.935 118.6624) (width 0.4) (layer "F.Cu") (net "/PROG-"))
 (segment locked (start 180.48 117.767) (end 175.9535 122.2935) (width 0.4) (layer "F.Cu") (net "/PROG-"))
 (segment locked (start 186.8402 115.0242) (end 183.2228 115.0242) (width 0.3) (layer "F.Cu") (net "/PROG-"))
 (segment locked (start 163.195 117.4022) (end 161.9348 118.6624) (width 0.4) (layer "F.Cu") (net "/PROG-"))
 (segment locked (start 183.2228 115.0242) (end 180.48 117.767) (width 0.3) (layer "F.Cu") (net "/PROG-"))
 (segment locked (start 175.9535 122.2935) (end 159.8254 122.2935) (width 0.4) (layer "F.Cu") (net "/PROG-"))
 (segment locked (start 162.6529 110.8319) (end 163.195 111.374) (width 0.4) (layer "F.Cu") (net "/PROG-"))
 (segment locked (start 163.195 111.374) (end 163.195 117.4022) (width 0.4) (layer "F.Cu") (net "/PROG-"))
 (segment locked (start 161.925 110.104) (end 161.925 97.4278) (width 0.4) (layer "B.Cu") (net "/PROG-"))
 (segment locked (start 151.8424 119.5698) (end 150.935 118.6624) (width 0.4) (layer "B.Cu") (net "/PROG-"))
 (segment locked (start 159.8254 122.2935) (end 157.1017 119.5698) (width 0.4) (layer "B.Cu") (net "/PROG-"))
 (segment locked (start 157.1017 119.5698) (end 151.8424 119.5698) (width 0.4) (layer "B.Cu") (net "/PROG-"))
 (segment locked (start 162.6529 110.8319) (end 161.925 110.104) (width 0.4) (layer "B.Cu") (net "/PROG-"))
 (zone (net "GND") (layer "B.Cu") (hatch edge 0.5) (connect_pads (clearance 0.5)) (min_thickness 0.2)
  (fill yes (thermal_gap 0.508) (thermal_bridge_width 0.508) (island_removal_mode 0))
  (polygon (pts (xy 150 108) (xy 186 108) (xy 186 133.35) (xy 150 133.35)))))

